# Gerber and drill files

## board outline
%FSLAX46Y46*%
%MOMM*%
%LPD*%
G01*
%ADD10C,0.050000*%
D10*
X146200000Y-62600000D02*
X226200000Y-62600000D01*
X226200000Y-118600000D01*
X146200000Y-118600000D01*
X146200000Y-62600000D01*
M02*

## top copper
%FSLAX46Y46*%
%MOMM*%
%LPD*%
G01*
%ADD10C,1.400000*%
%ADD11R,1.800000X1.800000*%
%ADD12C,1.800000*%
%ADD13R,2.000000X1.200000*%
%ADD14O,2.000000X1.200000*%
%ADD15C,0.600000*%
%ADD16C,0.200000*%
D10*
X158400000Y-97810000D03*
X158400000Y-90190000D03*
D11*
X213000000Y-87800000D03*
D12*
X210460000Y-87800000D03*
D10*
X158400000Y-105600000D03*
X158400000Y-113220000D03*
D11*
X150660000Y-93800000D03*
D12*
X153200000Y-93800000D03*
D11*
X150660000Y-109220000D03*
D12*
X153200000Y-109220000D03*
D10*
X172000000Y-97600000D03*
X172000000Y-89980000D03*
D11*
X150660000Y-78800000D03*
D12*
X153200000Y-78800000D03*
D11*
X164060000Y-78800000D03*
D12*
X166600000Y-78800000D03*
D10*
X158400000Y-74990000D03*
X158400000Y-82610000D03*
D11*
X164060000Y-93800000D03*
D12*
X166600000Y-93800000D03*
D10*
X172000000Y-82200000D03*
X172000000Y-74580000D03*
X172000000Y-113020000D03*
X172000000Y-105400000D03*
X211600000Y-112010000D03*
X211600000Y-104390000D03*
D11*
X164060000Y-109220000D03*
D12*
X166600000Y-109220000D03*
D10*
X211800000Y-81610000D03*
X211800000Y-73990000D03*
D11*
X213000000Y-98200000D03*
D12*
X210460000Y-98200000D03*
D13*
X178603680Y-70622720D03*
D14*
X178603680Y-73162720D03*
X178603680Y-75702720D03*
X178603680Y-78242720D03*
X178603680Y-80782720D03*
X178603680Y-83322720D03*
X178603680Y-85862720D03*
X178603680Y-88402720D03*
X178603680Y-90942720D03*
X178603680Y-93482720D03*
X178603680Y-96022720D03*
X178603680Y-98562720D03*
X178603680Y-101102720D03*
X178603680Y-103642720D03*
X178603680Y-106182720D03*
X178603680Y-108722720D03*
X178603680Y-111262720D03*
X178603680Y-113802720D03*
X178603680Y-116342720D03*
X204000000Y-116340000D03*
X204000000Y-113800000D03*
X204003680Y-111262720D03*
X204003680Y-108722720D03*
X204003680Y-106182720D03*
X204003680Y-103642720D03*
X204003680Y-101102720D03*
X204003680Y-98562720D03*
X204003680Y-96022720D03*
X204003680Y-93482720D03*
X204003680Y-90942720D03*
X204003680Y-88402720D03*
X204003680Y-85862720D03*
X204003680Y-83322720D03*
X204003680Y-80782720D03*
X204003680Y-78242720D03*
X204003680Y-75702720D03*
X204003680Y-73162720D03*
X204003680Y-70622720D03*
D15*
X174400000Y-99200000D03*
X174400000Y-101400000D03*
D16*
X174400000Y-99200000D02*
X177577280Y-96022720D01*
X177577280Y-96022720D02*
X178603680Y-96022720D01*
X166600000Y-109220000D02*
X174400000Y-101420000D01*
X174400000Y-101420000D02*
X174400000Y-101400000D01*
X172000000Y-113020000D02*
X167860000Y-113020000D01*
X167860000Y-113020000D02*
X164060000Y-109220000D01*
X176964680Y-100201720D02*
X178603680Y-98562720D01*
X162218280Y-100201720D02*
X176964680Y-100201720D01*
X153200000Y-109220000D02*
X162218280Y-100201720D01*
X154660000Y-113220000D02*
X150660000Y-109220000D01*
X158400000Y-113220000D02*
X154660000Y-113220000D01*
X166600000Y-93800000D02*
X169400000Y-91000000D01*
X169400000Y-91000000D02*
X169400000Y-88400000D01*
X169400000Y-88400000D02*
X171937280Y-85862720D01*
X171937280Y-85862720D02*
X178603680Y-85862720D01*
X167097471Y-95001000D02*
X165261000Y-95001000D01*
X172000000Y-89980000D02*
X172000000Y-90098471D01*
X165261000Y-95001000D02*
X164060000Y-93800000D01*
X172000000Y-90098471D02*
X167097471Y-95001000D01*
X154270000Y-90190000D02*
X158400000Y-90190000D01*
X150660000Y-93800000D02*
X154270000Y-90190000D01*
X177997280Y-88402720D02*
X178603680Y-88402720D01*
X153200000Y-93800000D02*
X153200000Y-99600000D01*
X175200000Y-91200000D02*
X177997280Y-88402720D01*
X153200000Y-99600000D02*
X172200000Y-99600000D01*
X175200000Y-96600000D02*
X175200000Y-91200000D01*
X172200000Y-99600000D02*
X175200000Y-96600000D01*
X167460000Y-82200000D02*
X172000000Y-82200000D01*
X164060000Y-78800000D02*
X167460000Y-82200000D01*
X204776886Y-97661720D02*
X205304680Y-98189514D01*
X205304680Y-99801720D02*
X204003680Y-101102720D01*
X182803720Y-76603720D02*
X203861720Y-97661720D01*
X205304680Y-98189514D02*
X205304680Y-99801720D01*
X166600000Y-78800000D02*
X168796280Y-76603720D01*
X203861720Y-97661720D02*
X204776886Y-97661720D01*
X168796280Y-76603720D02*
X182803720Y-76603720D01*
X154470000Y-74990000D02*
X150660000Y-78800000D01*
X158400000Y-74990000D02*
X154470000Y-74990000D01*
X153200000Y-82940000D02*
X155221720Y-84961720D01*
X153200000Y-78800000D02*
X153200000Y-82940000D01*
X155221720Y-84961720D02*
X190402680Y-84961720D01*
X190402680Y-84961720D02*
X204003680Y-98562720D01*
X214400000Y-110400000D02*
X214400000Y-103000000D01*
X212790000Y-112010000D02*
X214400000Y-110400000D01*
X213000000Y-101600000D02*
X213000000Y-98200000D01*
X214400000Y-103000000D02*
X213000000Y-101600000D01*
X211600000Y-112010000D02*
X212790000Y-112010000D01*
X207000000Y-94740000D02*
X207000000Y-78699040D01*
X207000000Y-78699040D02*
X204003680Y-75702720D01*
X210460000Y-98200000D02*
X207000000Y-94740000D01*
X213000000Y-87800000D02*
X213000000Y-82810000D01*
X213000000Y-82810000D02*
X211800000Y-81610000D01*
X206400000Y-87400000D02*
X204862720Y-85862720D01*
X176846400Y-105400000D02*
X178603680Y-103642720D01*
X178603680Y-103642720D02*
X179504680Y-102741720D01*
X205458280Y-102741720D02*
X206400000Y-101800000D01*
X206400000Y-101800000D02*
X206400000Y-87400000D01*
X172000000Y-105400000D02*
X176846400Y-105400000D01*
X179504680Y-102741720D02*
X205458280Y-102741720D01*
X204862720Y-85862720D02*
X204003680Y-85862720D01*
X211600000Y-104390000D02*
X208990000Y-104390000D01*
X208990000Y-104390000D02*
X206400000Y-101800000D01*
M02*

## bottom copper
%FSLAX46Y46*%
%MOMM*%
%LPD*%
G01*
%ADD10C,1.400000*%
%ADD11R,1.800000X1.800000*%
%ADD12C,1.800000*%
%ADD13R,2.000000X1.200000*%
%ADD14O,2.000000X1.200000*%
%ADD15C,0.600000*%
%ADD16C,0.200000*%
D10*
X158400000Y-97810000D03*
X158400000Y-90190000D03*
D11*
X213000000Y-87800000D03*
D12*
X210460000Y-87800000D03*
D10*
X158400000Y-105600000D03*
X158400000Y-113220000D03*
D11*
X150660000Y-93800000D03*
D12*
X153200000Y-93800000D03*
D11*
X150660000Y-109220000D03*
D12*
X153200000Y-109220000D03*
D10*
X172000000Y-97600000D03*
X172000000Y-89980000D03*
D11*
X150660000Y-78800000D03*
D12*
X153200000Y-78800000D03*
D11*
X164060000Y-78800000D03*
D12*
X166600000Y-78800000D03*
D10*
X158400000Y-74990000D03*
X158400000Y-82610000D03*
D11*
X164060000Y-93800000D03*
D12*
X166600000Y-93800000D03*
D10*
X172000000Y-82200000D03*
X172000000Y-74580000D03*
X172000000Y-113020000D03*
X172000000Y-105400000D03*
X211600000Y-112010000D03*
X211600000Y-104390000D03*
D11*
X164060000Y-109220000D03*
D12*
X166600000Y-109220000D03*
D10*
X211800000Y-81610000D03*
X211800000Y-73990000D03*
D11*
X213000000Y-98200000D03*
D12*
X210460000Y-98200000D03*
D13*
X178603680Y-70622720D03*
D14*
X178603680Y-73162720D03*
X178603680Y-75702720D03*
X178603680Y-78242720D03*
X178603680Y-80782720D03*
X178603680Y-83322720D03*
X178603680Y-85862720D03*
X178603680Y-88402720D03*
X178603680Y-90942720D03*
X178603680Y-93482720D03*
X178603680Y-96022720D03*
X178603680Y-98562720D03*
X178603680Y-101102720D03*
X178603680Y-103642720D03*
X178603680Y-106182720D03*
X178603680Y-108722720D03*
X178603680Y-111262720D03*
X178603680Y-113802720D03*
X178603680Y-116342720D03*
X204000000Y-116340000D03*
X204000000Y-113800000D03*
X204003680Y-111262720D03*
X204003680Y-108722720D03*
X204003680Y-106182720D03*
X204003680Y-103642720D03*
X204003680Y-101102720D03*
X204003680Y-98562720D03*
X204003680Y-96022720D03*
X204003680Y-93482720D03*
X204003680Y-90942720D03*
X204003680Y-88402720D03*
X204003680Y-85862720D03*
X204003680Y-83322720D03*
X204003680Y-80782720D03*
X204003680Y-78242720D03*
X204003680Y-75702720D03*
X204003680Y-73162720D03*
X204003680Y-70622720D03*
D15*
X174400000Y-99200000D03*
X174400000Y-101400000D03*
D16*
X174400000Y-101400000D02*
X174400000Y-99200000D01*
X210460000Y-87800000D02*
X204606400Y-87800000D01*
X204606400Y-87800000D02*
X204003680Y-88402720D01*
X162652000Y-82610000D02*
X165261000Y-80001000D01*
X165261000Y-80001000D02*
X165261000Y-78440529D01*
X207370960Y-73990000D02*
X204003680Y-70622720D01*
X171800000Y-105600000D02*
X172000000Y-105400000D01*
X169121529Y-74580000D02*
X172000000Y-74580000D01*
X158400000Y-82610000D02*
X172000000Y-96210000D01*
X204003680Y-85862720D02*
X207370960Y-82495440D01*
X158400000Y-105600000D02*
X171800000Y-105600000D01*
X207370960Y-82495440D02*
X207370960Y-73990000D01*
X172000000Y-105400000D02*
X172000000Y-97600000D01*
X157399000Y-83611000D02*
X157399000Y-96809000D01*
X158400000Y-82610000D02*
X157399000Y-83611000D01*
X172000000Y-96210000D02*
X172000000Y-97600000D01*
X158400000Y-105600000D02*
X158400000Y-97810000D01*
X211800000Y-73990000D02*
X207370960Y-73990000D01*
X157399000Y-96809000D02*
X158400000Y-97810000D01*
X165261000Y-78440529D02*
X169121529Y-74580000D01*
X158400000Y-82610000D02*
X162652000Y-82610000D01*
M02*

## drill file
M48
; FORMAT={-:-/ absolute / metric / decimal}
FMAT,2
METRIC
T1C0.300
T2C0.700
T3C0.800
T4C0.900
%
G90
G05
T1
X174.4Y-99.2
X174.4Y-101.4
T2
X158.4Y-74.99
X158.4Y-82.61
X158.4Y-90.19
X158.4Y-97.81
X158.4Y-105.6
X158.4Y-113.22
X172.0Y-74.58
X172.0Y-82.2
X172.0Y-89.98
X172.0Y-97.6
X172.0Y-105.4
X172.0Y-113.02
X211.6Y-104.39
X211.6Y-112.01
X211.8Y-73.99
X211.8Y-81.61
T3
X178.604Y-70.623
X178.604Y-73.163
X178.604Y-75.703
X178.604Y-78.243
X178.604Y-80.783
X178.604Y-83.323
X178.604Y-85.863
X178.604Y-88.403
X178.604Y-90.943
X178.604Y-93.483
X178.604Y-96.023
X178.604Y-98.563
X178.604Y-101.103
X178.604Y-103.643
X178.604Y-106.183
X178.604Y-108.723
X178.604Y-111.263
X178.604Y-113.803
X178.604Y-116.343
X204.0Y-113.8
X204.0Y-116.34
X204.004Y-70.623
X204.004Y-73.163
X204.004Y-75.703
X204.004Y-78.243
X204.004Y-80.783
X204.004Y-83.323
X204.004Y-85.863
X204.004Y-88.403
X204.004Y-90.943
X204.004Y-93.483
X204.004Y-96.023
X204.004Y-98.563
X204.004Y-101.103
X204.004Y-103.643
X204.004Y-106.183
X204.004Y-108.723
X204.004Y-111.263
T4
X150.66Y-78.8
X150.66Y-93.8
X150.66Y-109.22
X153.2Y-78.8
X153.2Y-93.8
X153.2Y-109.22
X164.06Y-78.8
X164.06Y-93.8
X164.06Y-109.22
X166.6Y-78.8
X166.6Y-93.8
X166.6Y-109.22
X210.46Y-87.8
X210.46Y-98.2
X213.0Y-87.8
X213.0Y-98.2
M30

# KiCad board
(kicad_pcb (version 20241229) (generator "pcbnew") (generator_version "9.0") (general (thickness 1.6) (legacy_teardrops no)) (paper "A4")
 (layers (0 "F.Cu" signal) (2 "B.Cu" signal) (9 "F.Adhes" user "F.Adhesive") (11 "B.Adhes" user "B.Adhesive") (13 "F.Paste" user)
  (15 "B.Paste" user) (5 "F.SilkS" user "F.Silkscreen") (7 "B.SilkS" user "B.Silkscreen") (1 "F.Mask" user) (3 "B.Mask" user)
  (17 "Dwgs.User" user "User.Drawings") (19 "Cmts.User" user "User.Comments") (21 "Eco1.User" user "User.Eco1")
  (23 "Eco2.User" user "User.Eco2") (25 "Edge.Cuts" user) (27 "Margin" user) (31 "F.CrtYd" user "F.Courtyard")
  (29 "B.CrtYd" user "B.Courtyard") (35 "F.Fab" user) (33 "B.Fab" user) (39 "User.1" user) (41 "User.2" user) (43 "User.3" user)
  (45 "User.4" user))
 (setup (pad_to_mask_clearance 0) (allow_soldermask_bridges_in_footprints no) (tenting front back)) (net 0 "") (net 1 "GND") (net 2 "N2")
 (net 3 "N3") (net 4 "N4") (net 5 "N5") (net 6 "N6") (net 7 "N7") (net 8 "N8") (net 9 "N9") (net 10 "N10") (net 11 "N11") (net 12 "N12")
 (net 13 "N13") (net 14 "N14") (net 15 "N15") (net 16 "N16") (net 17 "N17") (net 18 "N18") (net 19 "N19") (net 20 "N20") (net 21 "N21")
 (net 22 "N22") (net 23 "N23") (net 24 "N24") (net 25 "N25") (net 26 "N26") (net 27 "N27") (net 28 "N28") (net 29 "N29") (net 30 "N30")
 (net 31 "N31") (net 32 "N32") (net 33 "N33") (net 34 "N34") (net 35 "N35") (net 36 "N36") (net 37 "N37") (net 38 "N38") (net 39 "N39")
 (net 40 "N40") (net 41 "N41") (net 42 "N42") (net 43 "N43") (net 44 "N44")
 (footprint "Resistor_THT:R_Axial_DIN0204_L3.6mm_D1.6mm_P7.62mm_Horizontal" (layer "F.Cu") (at 158.4 97.81 90)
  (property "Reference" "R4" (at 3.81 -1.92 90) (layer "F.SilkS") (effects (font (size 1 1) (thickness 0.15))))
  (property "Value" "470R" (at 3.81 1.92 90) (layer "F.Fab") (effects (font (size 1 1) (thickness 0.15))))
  (pad "1" thru_hole circle (at 0 0 90) (size 1.4 1.4) (drill 0.7) (layers "*.Cu" "*.Mask") (remove_unused_layers no) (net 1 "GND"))
  (pad "2" thru_hole circle (at 7.62 0 90) (size 1.4 1.4) (drill 0.7) (layers "*.Cu" "*.Mask") (remove_unused_layers no) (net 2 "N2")))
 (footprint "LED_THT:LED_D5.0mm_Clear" (layer "F.Cu") (at 213 87.8 180)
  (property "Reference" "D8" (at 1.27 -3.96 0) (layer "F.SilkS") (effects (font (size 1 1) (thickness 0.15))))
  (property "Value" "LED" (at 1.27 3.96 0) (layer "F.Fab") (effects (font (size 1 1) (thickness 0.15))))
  (pad "1" thru_hole rect (at 0 0 180) (size 1.8 1.8) (drill 0.9) (layers "*.Cu" "*.Mask") (remove_unused_layers no) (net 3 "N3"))
  (pad "2" thru_hole circle (at 2.54 0 180) (size 1.8 1.8) (drill 0.9) (layers "*.Cu" "*.Mask") (remove_unused_layers no) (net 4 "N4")))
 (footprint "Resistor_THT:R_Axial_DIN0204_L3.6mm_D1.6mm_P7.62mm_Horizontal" (layer "F.Cu") (at 158.4 105.6 -90)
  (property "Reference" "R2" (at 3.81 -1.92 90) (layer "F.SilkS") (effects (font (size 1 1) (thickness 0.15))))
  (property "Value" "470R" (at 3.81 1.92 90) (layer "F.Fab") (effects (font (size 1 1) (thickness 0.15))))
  (pad "1" thru_hole circle (at 0 0 270) (size 1.4 1.4) (drill 0.7) (layers "*.Cu" "*.Mask") (remove_unused_layers no) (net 1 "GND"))
  (pad "2" thru_hole circle (at 7.62 0 270) (size 1.4 1.4) (drill 0.7) (layers "*.Cu" "*.Mask") (remove_unused_layers no) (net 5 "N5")))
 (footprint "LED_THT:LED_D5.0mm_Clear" (layer "F.Cu") (at 150.66 93.8)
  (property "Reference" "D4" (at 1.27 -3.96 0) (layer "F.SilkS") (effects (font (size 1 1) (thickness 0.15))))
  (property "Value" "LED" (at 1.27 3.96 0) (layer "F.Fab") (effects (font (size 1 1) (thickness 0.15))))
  (pad "1" thru_hole rect (at 0 0) (size 1.8 1.8) (drill 0.9) (layers "*.Cu" "*.Mask") (remove_unused_layers no) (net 2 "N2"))
  (pad "2" thru_hole circle (at 2.54 0) (size 1.8 1.8) (drill 0.9) (layers "*.Cu" "*.Mask") (remove_unused_layers no) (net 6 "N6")))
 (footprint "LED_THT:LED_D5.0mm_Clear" (layer "F.Cu") (at 150.66 109.22)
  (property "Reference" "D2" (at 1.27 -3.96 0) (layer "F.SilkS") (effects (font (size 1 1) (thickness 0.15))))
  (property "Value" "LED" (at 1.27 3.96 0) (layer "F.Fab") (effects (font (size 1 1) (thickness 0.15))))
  (pad "1" thru_hole rect (at 0 0) (size 1.8 1.8) (drill 0.9) (layers "*.Cu" "*.Mask") (remove_unused_layers no) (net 5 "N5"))
  (pad "2" thru_hole circle (at 2.54 0) (size 1.8 1.8) (drill 0.9) (layers "*.Cu" "*.Mask") (remove_unused_layers no) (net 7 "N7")))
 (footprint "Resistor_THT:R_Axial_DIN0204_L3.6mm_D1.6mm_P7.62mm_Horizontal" (layer "F.Cu") (at 172 97.6 90)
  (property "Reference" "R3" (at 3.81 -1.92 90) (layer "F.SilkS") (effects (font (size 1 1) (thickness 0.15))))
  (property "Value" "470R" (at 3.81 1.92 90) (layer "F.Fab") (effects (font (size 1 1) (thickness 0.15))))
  (pad "1" thru_hole circle (at 0 0 90) (size 1.4 1.4) (drill 0.7) (layers "*.Cu" "*.Mask") (remove_unused_layers no) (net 1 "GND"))
  (pad "2" thru_hole circle (at 7.62 0 90) (size 1.4 1.4) (drill 0.7) (layers "*.Cu" "*.Mask") (remove_unused_layers no) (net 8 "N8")))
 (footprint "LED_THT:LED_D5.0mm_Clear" (layer "F.Cu") (at 150.66 78.8)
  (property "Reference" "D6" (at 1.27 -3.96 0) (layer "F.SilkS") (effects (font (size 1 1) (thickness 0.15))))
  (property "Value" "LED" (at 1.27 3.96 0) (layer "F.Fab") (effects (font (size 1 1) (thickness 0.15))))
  (pad "1" thru_hole rect (at 0 0) (size 1.8 1.8) (drill 0.9) (layers "*.Cu" "*.Mask") (remove_unused_layers no) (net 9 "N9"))
  (pad "2" thru_hole circle (at 2.54 0) (size 1.8 1.8) (drill 0.9) (layers "*.Cu" "*.Mask") (remove_unused_layers no) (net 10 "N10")))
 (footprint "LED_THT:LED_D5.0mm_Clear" (layer "F.Cu") (at 164.06 78.8)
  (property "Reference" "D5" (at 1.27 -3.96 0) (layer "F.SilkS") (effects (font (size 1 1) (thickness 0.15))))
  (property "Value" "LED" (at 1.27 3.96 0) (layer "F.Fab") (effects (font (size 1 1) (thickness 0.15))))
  (pad "1" thru_hole rect (at 0 0) (size 1.8 1.8) (drill 0.9) (layers "*.Cu" "*.Mask") (remove_unused_layers no) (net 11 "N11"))
  (pad "2" thru_hole circle (at 2.54 0) (size 1.8 1.8) (drill 0.9) (layers "*.Cu" "*.Mask") (remove_unused_layers no) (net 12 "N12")))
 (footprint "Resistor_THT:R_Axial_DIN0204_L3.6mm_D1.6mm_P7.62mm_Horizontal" (layer "F.Cu") (at 158.4 74.99 -90)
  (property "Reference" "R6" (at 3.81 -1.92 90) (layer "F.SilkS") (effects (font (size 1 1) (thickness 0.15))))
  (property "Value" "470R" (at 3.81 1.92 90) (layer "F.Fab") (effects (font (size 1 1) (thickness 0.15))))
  (pad "1" thru_hole circle (at 0 0 270) (size 1.4 1.4) (drill 0.7) (layers "*.Cu" "*.Mask") (remove_unused_layers no) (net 9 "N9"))
  (pad "2" thru_hole circle (at 7.62 0 270) (size 1.4 1.4) (drill 0.7) (layers "*.Cu" "*.Mask") (remove_unused_layers no) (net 1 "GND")))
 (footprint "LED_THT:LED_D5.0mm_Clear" (layer "F.Cu") (at 164.06 93.8)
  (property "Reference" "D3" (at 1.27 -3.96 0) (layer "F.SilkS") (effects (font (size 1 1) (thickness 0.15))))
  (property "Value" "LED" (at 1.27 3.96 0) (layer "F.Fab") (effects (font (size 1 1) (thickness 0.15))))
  (pad "1" thru_hole rect (at 0 0) (size 1.8 1.8) (drill 0.9) (layers "*.Cu" "*.Mask") (remove_unused_layers no) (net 8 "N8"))
  (pad "2" thru_hole circle (at 2.54 0) (size 1.8 1.8) (drill 0.9) (layers "*.Cu" "*.Mask") (remove_unused_layers no) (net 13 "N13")))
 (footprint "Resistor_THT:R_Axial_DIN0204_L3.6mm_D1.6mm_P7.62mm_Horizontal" (layer "F.Cu") (at 172 82.2 90)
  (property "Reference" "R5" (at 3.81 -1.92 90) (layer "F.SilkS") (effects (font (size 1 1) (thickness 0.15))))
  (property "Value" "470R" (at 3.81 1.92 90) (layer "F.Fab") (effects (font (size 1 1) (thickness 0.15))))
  (pad "1" thru_hole circle (at 0 0 90) (size 1.4 1.4) (drill 0.7) (layers "*.Cu" "*.Mask") (remove_unused_layers no) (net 11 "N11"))
  (pad "2" thru_hole circle (at 7.62 0 90) (size 1.4 1.4) (drill 0.7) (layers "*.Cu" "*.Mask") (remove_unused_layers no) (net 1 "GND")))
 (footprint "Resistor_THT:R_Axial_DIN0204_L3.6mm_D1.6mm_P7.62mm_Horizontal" (layer "F.Cu") (at 172 113.02 90)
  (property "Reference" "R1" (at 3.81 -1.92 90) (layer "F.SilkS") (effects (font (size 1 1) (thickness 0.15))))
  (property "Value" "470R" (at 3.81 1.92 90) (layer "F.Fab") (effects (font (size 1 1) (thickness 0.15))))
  (pad "1" thru_hole circle (at 0 0 90) (size 1.4 1.4) (drill 0.7) (layers "*.Cu" "*.Mask") (remove_unused_layers no) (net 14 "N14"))
  (pad "2" thru_hole circle (at 7.62 0 90) (size 1.4 1.4) (drill 0.7) (layers "*.Cu" "*.Mask") (remove_unused_layers no) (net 1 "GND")))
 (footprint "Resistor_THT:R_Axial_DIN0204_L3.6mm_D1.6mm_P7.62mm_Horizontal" (layer "F.Cu") (at 211.6 112.01 90)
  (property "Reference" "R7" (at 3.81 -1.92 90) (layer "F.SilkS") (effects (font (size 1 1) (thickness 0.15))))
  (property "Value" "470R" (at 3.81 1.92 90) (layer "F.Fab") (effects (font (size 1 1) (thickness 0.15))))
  (pad "1" thru_hole circle (at 0 0 90) (size 1.4 1.4) (drill 0.7) (layers "*.Cu" "*.Mask") (remove_unused_layers no) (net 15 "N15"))
  (pad "2" thru_hole circle (at 7.62 0 90) (size 1.4 1.4) (drill 0.7) (layers "*.Cu" "*.Mask") (remove_unused_layers no) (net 1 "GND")))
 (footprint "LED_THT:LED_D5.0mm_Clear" (layer "F.Cu") (at 164.06 109.22)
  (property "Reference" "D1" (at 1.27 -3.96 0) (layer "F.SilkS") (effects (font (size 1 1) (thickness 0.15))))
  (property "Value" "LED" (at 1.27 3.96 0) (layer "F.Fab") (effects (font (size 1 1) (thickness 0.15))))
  (pad "1" thru_hole rect (at 0 0) (size 1.8 1.8) (drill 0.9) (layers "*.Cu" "*.Mask") (remove_unused_layers no) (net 14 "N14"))
  (pad "2" thru_hole circle (at 2.54 0) (size 1.8 1.8) (drill 0.9) (layers "*.Cu" "*.Mask") (remove_unused_layers no) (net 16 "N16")))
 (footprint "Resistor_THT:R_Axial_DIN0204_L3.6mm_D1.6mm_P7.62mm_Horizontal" (layer "F.Cu") (at 211.8 81.61 90)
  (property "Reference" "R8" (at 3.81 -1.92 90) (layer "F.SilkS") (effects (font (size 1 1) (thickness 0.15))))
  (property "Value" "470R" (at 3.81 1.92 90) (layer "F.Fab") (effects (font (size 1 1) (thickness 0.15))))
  (pad "1" thru_hole circle (at 0 0 90) (size 1.4 1.4) (drill 0.7) (layers "*.Cu" "*.Mask") (remove_unused_layers no) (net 3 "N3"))
  (pad "2" thru_hole circle (at 7.62 0 90) (size 1.4 1.4) (drill 0.7) (layers "*.Cu" "*.Mask") (remove_unused_layers no) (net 1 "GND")))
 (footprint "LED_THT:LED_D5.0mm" (layer "F.Cu") (at 213 98.2 180)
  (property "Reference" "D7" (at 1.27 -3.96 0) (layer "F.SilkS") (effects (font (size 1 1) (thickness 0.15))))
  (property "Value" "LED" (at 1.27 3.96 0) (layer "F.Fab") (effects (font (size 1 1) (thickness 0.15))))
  (pad "1" thru_hole rect (at 0 0 180) (size 1.8 1.8) (drill 0.9) (layers "*.Cu" "*.Mask") (remove_unused_layers no) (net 15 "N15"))
  (pad "2" thru_hole circle (at 2.54 0 180) (size 1.8 1.8) (drill 0.9) (layers "*.Cu" "*.Mask") (remove_unused_layers no) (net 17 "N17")))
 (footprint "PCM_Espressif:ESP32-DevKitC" (layer "F.Cu") (at 178.60368 70.62272)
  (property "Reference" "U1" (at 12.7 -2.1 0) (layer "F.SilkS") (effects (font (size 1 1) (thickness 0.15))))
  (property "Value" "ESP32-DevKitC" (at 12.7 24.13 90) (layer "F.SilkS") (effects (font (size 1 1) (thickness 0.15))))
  (pad "1" thru_hole rect (at 0 0 270) (size 1.2 2) (drill 0.8) (layers "*.Cu" "*.Mask") (remove_unused_layers no) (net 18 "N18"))
  (pad "2" thru_hole oval (at 0 2.54 270) (size 1.2 2) (drill 0.8) (layers "*.Cu" "*.Mask") (remove_unused_layers no) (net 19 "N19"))
  (pad "3" thru_hole oval (at 0 5.08 270) (size 1.2 2) (drill 0.8) (layers "*.Cu" "*.Mask") (remove_unused_layers no) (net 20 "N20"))
  (pad "4" thru_hole oval (at 0 7.62 270) (size 1.2 2) (drill 0.8) (layers "*.Cu" "*.Mask") (remove_unused_layers no) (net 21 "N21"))
  (pad "5" thru_hole oval (at 0 10.16 270) (size 1.2 2) (drill 0.8) (layers "*.Cu" "*.Mask") (remove_unused_layers no) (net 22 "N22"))
  (pad "6" thru_hole oval (at 0 12.7 270) (size 1.2 2) (drill 0.8) (layers "*.Cu" "*.Mask") (remove_unused_layers no) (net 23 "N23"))
  (pad "7" thru_hole oval (at 0 15.24 270) (size 1.2 2) (drill 0.8) (layers "*.Cu" "*.Mask") (remove_unused_layers no) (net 13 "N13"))
  (pad "8" thru_hole oval (at 0 17.78 270) (size 1.2 2) (drill 0.8) (layers "*.Cu" "*.Mask") (remove_unused_layers no) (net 6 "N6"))
  (pad "9" thru_hole oval (at 0 20.32 270) (size 1.2 2) (drill 0.8) (layers "*.Cu" "*.Mask") (remove_unused_layers no) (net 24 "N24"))
  (pad "10" thru_hole oval (at 0 22.86 270) (size 1.2 2) (drill 0.8) (layers "*.Cu" "*.Mask") (remove_unused_layers no) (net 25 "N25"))
  (pad "11" thru_hole oval (at 0 25.4 270) (size 1.2 2) (drill 0.8) (layers "*.Cu" "*.Mask") (remove_unused_layers no) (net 16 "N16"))
  (pad "12" thru_hole oval (at 0 27.94 270) (size 1.2 2) (drill 0.8) (layers "*.Cu" "*.Mask") (remove_unused_layers no) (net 7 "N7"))
  (pad "13" thru_hole oval (at 0 30.48 270) (size 1.2 2) (drill 0.8) (layers "*.Cu" "*.Mask") (remove_unused_layers no) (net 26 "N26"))
  (pad "14" thru_hole oval (at 0 33.02 270) (size 1.2 2) (drill 0.8) (layers "*.Cu" "*.Mask") (remove_unused_layers no) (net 1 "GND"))
  (pad "15" thru_hole oval (at 0 35.56 270) (size 1.2 2) (drill 0.8) (layers "*.Cu" "*.Mask") (remove_unused_layers no) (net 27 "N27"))
  (pad "16" thru_hole oval (at 0 38.1 270) (size 1.2 2) (drill 0.8) (layers "*.Cu" "*.Mask") (remove_unused_layers no) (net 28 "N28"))
  (pad "17" thru_hole oval (at 0 40.64 270) (size 1.2 2) (drill 0.8) (layers "*.Cu" "*.Mask") (remove_unused_layers no) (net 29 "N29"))
  (pad "18" thru_hole oval (at 0 43.18 270) (size 1.2 2) (drill 0.8) (layers "*.Cu" "*.Mask") (remove_unused_layers no) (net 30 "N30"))
  (pad "19" thru_hole oval (at 0 45.72 270) (size 1.2 2) (drill 0.8) (layers "*.Cu" "*.Mask") (remove_unused_layers no) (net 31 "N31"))
  (pad "20" thru_hole oval (at 25.39632 45.71728 270) (size 1.2 2) (drill 0.8) (layers "*.Cu" "*.Mask") (remove_unused_layers no)
   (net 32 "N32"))
  (pad "21" thru_hole oval (at 25.39632 43.17728 270) (size 1.2 2) (drill 0.8) (layers "*.Cu" "*.Mask") (remove_unused_layers no)
   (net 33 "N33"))
  (pad "22" thru_hole oval (at 25.4 40.64 270) (size 1.2 2) (drill 0.8) (layers "*.Cu" "*.Mask") (remove_unused_layers no) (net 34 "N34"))
  (pad "23" thru_hole oval (at 25.4 38.1 270) (size 1.2 2) (drill 0.8) (layers "*.Cu" "*.Mask") (remove_unused_layers no) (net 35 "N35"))
  (pad "24" thru_hole oval (at 25.4 35.56 270) (size 1.2 2) (drill 0.8) (layers "*.Cu" "*.Mask") (remove_unused_layers no) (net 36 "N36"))
  (pad "25" thru_hole oval (at 25.4 33.02 270) (size 1.2 2) (drill 0.8) (layers "*.Cu" "*.Mask") (remove_unused_layers no) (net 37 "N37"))
  (pad "26" thru_hole oval (at 25.4 30.48 270) (size 1.2 2) (drill 0.8) (layers "*.Cu" "*.Mask") (remove_unused_layers no) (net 12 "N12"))
  (pad "27" thru_hole oval (at 25.4 27.94 270) (size 1.2 2) (drill 0.8) (layers "*.Cu" "*.Mask") (remove_unused_layers no) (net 10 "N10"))
  (pad "28" thru_hole oval (at 25.4 25.4 270) (size 1.2 2) (drill 0.8) (layers "*.Cu" "*.Mask") (remove_unused_layers no) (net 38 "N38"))
  (pad "29" thru_hole oval (at 25.4 22.86 270) (size 1.2 2) (drill 0.8) (layers "*.Cu" "*.Mask") (remove_unused_layers no) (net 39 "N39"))
  (pad "30" thru_hole oval (at 25.4 20.32 270) (size 1.2 2) (drill 0.8) (layers "*.Cu" "*.Mask") (remove_unused_layers no) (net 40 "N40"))
  (pad "31" thru_hole oval (at 25.4 17.78 270) (size 1.2 2) (drill 0.8) (layers "*.Cu" "*.Mask") (remove_unused_layers no) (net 4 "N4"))
  (pad "32" thru_hole oval (at 25.4 15.24 270) (size 1.2 2) (drill 0.8) (layers "*.Cu" "*.Mask") (remove_unused_layers no) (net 1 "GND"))
  (pad "33" thru_hole oval (at 25.4 12.7 270) (size 1.2 2) (drill 0.8) (layers "*.Cu" "*.Mask") (remove_unused_layers no) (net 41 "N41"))
  (pad "34" thru_hole oval (at 25.4 10.16 270) (size 1.2 2) (drill 0.8) (layers "*.Cu" "*.Mask") (remove_unused_layers no) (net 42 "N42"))
  (pad "35" thru_hole oval (at 25.4 7.62 270) (size 1.2 2) (drill 0.8) (layers "*.Cu" "*.Mask") (remove_unused_layers no) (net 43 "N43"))
  (pad "36" thru_hole oval (at 25.4 5.08 270) (size 1.2 2) (drill 0.8) (layers "*.Cu" "*.Mask") (remove_unused_layers no) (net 17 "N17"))
  (pad "37" thru_hole oval (at 25.4 2.54 270) (size 1.2 2) (drill 0.8) (layers "*.Cu" "*.Mask") (remove_unused_layers no) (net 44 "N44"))
  (pad "38" thru_hole oval (at 25.4 0 270) (size 1.2 2) (drill 0.8) (layers "*.Cu" "*.Mask") (remove_unused_layers no) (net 1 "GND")))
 (gr_rect (start 146.2 62.6) (end 226.2 118.6) (stroke (width 0.05) (type default)) (fill no) (layer "Edge.Cuts"))
 (segment (start 174.4 99.2) (end 177.57728 96.02272) (width 0.2) (layer "F.Cu") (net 16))
 (segment (start 177.57728 96.02272) (end 178.60368 96.02272) (width 0.2) (layer "F.Cu") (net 16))
 (segment (start 166.6 109.22) (end 174.4 101.42) (width 0.2) (layer "F.Cu") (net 16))
 (segment (start 174.4 101.42) (end 174.4 101.4) (width 0.2) (layer "F.Cu") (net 16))
 (via (at 174.4 99.2) (size 0.6) (drill 0.3) (layers "F.Cu" "B.Cu") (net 16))
 (via (at 174.4 101.4) (size 0.6) (drill 0.3) (layers "F.Cu" "B.Cu") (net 16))
 (segment (start 174.4 101.4) (end 174.4 99.2) (width 0.2) (layer "B.Cu") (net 16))
 (segment (start 172 113.02) (end 167.86 113.02) (width 0.2) (layer "F.Cu") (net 14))
 (segment (start 167.86 113.02) (end 164.06 109.22) (width 0.2) (layer "F.Cu") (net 14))
 (segment (start 176.96468 100.20172) (end 178.60368 98.56272) (width 0.2) (layer "F.Cu") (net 7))
 (segment (start 162.21828 100.20172) (end 176.96468 100.20172) (width 0.2) (layer "F.Cu") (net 7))
 (segment (start 153.2 109.22) (end 162.21828 100.20172) (width 0.2) (layer "F.Cu") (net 7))
 (segment (start 154.66 113.22) (end 150.66 109.22) (width 0.2) (layer "F.Cu") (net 5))
 (segment (start 158.4 113.22) (end 154.66 113.22) (width 0.2) (layer "F.Cu") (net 5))
 (segment (start 166.6 93.8) (end 169.4 91) (width 0.2) (layer "F.Cu") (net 13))
 (segment (start 169.4 91) (end 169.4 88.4) (width 0.2) (layer "F.Cu") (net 13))
 (segment (start 169.4 88.4) (end 171.93728 85.86272) (width 0.2) (layer "F.Cu") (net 13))
 (segment (start 171.93728 85.86272) (end 178.60368 85.86272) (width 0.2) (layer "F.Cu") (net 13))
 (segment (start 167.097471 95.001) (end 165.261 95.001) (width 0.2) (layer "F.Cu") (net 8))
 (segment (start 172 89.98) (end 172 90.098471) (width 0.2) (layer "F.Cu") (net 8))
 (segment (start 165.261 95.001) (end 164.06 93.8) (width 0.2) (layer "F.Cu") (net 8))
 (segment (start 172 90.098471) (end 167.097471 95.001) (width 0.2) (layer "F.Cu") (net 8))
 (segment (start 154.27 90.19) (end 158.4 90.19) (width 0.2) (layer "F.Cu") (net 2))
 (segment (start 150.66 93.8) (end 154.27 90.19) (width 0.2) (layer "F.Cu") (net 2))
 (segment (start 177.99728 88.40272) (end 178.60368 88.40272) (width 0.2) (layer "F.Cu") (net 6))
 (segment (start 153.2 93.8) (end 153.2 99.6) (width 0.2) (layer "F.Cu") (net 6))
 (segment (start 175.2 91.2) (end 177.99728 88.40272) (width 0.2) (layer "F.Cu") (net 6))
 (segment (start 153.2 99.6) (end 172.2 99.6) (width 0.2) (layer "F.Cu") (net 6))
 (segment (start 175.2 96.6) (end 175.2 91.2) (width 0.2) (layer "F.Cu") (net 6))
 (segment (start 172.2 99.6) (end 175.2 96.6) (width 0.2) (layer "F.Cu") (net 6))
 (segment (start 167.46 82.2) (end 172 82.2) (width 0.2) (layer "F.Cu") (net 11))
 (segment (start 164.06 78.8) (end 167.46 82.2) (width 0.2) (layer "F.Cu") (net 11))
 (segment (start 204.776886 97.66172) (end 205.30468 98.189514) (width 0.2) (layer "F.Cu") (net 12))
 (segment (start 205.30468 99.80172) (end 204.00368 101.10272) (width 0.2) (layer "F.Cu") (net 12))
 (segment (start 182.80372 76.60372) (end 203.86172 97.66172) (width 0.2) (layer "F.Cu") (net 12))
 (segment (start 205.30468 98.189514) (end 205.30468 99.80172) (width 0.2) (layer "F.Cu") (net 12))
 (segment (start 166.6 78.8) (end 168.79628 76.60372) (width 0.2) (layer "F.Cu") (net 12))
 (segment (start 203.86172 97.66172) (end 204.776886 97.66172) (width 0.2) (layer "F.Cu") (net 12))
 (segment (start 168.79628 76.60372) (end 182.80372 76.60372) (width 0.2) (layer "F.Cu") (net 12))
 (segment (start 154.47 74.99) (end 150.66 78.8) (width 0.2) (layer "F.Cu") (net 9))
 (segment (start 158.4 74.99) (end 154.47 74.99) (width 0.2) (layer "F.Cu") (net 9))
 (segment (start 153.2 82.94) (end 155.22172 84.96172) (width 0.2) (layer "F.Cu") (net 10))
 (segment (start 153.2 78.8) (end 153.2 82.94) (width 0.2) (layer "F.Cu") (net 10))
 (segment (start 155.22172 84.96172) (end 190.40268 84.96172) (width 0.2) (layer "F.Cu") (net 10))
 (segment (start 190.40268 84.96172) (end 204.00368 98.56272) (width 0.2) (layer "F.Cu") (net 10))
 (segment (start 214.4 110.4) (end 214.4 103) (width 0.2) (layer "F.Cu") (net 15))
 (segment (start 212.79 112.01) (end 214.4 110.4) (width 0.2) (layer "F.Cu") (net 15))
 (segment (start 213 101.6) (end 213 98.2) (width 0.2) (layer "F.Cu") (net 15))
 (segment (start 214.4 103) (end 213 101.6) (width 0.2) (layer "F.Cu") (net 15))
 (segment (start 211.6 112.01) (end 212.79 112.01) (width 0.2) (layer "F.Cu") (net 15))
 (segment (start 207 94.74) (end 207 78.69904) (width 0.2) (layer "F.Cu") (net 17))
 (segment (start 207 78.69904) (end 204.00368 75.70272) (width 0.2) (layer "F.Cu") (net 17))
 (segment (start 210.46 98.2) (end 207 94.74) (width 0.2) (layer "F.Cu") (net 17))
 (segment (start 213 87.8) (end 213 82.81) (width 0.2) (layer "F.Cu") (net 3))
 (segment (start 213 82.81) (end 211.8 81.61) (width 0.2) (layer "F.Cu") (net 3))
 (segment (start 210.46 87.8) (end 204.6064 87.8) (width 0.2) (layer "B.Cu") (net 4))
 (segment (start 204.6064 87.8) (end 204.00368 88.40272) (width 0.2) (layer "B.Cu") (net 4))
 (segment (start 206.4 87.4) (end 204.86272 85.86272) (width 0.2) (layer "F.Cu") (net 1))
 (segment (start 176.8464 105.4) (end 178.60368 103.64272) (width 0.2) (layer "F.Cu") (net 1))
 (segment (start 178.60368 103.64272) (end 179.50468 102.74172) (width 0.2) (layer "F.Cu") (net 1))
 (segment (start 205.45828 102.74172) (end 206.4 101.8) (width 0.2) (layer "F.Cu") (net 1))
 (segment (start 206.4 101.8) (end 206.4 87.4) (width 0.2) (layer "F.Cu") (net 1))
 (segment (start 172 105.4) (end 176.8464 105.4) (width 0.2) (layer "F.Cu") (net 1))
 (segment (start 179.50468 102.74172) (end 205.45828 102.74172) (width 0.2) (layer "F.Cu") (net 1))
 (segment (start 204.86272 85.86272) (end 204.00368 85.86272) (width 0.2) (layer "F.Cu") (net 1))
 (segment (start 211.6 104.39) (end 208.99 104.39) (width 0.2) (layer "F.Cu") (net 1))
 (segment (start 208.99 104.39) (end 206.4 101.8) (width 0.2) (layer "F.Cu") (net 1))
 (segment (start 162.652 82.61) (end 165.261 80.001) (width 0.2) (layer "B.Cu") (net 1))
 (segment (start 165.261 80.001) (end 165.261 78.440529) (width 0.2) (layer "B.Cu") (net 1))
 (segment (start 207.37096 73.99) (end 204.00368 70.62272) (width 0.2) (layer "B.Cu") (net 1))
 (segment (start 171.8 105.6) (end 172 105.4) (width 0.2) (layer "B.Cu") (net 1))
 (segment (start 169.121529 74.58) (end 172 74.58) (width 0.2) (layer "B.Cu") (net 1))
 (segment (start 158.4 82.61) (end 172 96.21) (width 0.2) (layer "B.Cu") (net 1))
 (segment (start 204.00368 85.86272) (end 207.37096 82.49544) (width 0.2) (layer "B.Cu") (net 1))
 (segment (start 158.4 105.6) (end 171.8 105.6) (width 0.2) (layer "B.Cu") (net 1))
 (segment (start 207.37096 82.49544) (end 207.37096 73.99) (width 0.2) (layer "B.Cu") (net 1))
 (segment (start 172 105.4) (end 172 97.6) (width 0.2) (layer "B.Cu") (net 1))
 (segment (start 157.399 83.611) (end 157.399 96.809) (width 0.2) (layer "B.Cu") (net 1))
 (segment (start 158.4 82.61) (end 157.399 83.611) (width 0.2) (layer "B.Cu") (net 1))
 (segment (start 172 96.21) (end 172 97.6) (width 0.2) (layer "B.Cu") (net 1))
 (segment (start 158.4 105.6) (end 158.4 97.81) (width 0.2) (layer "B.Cu") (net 1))
 (segment (start 211.8 73.99) (end 207.37096 73.99) (width 0.2) (layer "B.Cu") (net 1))
 (segment (start 157.399 96.809) (end 158.4 97.81) (width 0.2) (layer "B.Cu") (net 1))
 (segment (start 165.261 78.440529) (end 169.121529 74.58) (width 0.2) (layer "B.Cu") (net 1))
 (segment (start 158.4 82.61) (end 162.652 82.61) (width 0.2) (layer "B.Cu") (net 1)))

